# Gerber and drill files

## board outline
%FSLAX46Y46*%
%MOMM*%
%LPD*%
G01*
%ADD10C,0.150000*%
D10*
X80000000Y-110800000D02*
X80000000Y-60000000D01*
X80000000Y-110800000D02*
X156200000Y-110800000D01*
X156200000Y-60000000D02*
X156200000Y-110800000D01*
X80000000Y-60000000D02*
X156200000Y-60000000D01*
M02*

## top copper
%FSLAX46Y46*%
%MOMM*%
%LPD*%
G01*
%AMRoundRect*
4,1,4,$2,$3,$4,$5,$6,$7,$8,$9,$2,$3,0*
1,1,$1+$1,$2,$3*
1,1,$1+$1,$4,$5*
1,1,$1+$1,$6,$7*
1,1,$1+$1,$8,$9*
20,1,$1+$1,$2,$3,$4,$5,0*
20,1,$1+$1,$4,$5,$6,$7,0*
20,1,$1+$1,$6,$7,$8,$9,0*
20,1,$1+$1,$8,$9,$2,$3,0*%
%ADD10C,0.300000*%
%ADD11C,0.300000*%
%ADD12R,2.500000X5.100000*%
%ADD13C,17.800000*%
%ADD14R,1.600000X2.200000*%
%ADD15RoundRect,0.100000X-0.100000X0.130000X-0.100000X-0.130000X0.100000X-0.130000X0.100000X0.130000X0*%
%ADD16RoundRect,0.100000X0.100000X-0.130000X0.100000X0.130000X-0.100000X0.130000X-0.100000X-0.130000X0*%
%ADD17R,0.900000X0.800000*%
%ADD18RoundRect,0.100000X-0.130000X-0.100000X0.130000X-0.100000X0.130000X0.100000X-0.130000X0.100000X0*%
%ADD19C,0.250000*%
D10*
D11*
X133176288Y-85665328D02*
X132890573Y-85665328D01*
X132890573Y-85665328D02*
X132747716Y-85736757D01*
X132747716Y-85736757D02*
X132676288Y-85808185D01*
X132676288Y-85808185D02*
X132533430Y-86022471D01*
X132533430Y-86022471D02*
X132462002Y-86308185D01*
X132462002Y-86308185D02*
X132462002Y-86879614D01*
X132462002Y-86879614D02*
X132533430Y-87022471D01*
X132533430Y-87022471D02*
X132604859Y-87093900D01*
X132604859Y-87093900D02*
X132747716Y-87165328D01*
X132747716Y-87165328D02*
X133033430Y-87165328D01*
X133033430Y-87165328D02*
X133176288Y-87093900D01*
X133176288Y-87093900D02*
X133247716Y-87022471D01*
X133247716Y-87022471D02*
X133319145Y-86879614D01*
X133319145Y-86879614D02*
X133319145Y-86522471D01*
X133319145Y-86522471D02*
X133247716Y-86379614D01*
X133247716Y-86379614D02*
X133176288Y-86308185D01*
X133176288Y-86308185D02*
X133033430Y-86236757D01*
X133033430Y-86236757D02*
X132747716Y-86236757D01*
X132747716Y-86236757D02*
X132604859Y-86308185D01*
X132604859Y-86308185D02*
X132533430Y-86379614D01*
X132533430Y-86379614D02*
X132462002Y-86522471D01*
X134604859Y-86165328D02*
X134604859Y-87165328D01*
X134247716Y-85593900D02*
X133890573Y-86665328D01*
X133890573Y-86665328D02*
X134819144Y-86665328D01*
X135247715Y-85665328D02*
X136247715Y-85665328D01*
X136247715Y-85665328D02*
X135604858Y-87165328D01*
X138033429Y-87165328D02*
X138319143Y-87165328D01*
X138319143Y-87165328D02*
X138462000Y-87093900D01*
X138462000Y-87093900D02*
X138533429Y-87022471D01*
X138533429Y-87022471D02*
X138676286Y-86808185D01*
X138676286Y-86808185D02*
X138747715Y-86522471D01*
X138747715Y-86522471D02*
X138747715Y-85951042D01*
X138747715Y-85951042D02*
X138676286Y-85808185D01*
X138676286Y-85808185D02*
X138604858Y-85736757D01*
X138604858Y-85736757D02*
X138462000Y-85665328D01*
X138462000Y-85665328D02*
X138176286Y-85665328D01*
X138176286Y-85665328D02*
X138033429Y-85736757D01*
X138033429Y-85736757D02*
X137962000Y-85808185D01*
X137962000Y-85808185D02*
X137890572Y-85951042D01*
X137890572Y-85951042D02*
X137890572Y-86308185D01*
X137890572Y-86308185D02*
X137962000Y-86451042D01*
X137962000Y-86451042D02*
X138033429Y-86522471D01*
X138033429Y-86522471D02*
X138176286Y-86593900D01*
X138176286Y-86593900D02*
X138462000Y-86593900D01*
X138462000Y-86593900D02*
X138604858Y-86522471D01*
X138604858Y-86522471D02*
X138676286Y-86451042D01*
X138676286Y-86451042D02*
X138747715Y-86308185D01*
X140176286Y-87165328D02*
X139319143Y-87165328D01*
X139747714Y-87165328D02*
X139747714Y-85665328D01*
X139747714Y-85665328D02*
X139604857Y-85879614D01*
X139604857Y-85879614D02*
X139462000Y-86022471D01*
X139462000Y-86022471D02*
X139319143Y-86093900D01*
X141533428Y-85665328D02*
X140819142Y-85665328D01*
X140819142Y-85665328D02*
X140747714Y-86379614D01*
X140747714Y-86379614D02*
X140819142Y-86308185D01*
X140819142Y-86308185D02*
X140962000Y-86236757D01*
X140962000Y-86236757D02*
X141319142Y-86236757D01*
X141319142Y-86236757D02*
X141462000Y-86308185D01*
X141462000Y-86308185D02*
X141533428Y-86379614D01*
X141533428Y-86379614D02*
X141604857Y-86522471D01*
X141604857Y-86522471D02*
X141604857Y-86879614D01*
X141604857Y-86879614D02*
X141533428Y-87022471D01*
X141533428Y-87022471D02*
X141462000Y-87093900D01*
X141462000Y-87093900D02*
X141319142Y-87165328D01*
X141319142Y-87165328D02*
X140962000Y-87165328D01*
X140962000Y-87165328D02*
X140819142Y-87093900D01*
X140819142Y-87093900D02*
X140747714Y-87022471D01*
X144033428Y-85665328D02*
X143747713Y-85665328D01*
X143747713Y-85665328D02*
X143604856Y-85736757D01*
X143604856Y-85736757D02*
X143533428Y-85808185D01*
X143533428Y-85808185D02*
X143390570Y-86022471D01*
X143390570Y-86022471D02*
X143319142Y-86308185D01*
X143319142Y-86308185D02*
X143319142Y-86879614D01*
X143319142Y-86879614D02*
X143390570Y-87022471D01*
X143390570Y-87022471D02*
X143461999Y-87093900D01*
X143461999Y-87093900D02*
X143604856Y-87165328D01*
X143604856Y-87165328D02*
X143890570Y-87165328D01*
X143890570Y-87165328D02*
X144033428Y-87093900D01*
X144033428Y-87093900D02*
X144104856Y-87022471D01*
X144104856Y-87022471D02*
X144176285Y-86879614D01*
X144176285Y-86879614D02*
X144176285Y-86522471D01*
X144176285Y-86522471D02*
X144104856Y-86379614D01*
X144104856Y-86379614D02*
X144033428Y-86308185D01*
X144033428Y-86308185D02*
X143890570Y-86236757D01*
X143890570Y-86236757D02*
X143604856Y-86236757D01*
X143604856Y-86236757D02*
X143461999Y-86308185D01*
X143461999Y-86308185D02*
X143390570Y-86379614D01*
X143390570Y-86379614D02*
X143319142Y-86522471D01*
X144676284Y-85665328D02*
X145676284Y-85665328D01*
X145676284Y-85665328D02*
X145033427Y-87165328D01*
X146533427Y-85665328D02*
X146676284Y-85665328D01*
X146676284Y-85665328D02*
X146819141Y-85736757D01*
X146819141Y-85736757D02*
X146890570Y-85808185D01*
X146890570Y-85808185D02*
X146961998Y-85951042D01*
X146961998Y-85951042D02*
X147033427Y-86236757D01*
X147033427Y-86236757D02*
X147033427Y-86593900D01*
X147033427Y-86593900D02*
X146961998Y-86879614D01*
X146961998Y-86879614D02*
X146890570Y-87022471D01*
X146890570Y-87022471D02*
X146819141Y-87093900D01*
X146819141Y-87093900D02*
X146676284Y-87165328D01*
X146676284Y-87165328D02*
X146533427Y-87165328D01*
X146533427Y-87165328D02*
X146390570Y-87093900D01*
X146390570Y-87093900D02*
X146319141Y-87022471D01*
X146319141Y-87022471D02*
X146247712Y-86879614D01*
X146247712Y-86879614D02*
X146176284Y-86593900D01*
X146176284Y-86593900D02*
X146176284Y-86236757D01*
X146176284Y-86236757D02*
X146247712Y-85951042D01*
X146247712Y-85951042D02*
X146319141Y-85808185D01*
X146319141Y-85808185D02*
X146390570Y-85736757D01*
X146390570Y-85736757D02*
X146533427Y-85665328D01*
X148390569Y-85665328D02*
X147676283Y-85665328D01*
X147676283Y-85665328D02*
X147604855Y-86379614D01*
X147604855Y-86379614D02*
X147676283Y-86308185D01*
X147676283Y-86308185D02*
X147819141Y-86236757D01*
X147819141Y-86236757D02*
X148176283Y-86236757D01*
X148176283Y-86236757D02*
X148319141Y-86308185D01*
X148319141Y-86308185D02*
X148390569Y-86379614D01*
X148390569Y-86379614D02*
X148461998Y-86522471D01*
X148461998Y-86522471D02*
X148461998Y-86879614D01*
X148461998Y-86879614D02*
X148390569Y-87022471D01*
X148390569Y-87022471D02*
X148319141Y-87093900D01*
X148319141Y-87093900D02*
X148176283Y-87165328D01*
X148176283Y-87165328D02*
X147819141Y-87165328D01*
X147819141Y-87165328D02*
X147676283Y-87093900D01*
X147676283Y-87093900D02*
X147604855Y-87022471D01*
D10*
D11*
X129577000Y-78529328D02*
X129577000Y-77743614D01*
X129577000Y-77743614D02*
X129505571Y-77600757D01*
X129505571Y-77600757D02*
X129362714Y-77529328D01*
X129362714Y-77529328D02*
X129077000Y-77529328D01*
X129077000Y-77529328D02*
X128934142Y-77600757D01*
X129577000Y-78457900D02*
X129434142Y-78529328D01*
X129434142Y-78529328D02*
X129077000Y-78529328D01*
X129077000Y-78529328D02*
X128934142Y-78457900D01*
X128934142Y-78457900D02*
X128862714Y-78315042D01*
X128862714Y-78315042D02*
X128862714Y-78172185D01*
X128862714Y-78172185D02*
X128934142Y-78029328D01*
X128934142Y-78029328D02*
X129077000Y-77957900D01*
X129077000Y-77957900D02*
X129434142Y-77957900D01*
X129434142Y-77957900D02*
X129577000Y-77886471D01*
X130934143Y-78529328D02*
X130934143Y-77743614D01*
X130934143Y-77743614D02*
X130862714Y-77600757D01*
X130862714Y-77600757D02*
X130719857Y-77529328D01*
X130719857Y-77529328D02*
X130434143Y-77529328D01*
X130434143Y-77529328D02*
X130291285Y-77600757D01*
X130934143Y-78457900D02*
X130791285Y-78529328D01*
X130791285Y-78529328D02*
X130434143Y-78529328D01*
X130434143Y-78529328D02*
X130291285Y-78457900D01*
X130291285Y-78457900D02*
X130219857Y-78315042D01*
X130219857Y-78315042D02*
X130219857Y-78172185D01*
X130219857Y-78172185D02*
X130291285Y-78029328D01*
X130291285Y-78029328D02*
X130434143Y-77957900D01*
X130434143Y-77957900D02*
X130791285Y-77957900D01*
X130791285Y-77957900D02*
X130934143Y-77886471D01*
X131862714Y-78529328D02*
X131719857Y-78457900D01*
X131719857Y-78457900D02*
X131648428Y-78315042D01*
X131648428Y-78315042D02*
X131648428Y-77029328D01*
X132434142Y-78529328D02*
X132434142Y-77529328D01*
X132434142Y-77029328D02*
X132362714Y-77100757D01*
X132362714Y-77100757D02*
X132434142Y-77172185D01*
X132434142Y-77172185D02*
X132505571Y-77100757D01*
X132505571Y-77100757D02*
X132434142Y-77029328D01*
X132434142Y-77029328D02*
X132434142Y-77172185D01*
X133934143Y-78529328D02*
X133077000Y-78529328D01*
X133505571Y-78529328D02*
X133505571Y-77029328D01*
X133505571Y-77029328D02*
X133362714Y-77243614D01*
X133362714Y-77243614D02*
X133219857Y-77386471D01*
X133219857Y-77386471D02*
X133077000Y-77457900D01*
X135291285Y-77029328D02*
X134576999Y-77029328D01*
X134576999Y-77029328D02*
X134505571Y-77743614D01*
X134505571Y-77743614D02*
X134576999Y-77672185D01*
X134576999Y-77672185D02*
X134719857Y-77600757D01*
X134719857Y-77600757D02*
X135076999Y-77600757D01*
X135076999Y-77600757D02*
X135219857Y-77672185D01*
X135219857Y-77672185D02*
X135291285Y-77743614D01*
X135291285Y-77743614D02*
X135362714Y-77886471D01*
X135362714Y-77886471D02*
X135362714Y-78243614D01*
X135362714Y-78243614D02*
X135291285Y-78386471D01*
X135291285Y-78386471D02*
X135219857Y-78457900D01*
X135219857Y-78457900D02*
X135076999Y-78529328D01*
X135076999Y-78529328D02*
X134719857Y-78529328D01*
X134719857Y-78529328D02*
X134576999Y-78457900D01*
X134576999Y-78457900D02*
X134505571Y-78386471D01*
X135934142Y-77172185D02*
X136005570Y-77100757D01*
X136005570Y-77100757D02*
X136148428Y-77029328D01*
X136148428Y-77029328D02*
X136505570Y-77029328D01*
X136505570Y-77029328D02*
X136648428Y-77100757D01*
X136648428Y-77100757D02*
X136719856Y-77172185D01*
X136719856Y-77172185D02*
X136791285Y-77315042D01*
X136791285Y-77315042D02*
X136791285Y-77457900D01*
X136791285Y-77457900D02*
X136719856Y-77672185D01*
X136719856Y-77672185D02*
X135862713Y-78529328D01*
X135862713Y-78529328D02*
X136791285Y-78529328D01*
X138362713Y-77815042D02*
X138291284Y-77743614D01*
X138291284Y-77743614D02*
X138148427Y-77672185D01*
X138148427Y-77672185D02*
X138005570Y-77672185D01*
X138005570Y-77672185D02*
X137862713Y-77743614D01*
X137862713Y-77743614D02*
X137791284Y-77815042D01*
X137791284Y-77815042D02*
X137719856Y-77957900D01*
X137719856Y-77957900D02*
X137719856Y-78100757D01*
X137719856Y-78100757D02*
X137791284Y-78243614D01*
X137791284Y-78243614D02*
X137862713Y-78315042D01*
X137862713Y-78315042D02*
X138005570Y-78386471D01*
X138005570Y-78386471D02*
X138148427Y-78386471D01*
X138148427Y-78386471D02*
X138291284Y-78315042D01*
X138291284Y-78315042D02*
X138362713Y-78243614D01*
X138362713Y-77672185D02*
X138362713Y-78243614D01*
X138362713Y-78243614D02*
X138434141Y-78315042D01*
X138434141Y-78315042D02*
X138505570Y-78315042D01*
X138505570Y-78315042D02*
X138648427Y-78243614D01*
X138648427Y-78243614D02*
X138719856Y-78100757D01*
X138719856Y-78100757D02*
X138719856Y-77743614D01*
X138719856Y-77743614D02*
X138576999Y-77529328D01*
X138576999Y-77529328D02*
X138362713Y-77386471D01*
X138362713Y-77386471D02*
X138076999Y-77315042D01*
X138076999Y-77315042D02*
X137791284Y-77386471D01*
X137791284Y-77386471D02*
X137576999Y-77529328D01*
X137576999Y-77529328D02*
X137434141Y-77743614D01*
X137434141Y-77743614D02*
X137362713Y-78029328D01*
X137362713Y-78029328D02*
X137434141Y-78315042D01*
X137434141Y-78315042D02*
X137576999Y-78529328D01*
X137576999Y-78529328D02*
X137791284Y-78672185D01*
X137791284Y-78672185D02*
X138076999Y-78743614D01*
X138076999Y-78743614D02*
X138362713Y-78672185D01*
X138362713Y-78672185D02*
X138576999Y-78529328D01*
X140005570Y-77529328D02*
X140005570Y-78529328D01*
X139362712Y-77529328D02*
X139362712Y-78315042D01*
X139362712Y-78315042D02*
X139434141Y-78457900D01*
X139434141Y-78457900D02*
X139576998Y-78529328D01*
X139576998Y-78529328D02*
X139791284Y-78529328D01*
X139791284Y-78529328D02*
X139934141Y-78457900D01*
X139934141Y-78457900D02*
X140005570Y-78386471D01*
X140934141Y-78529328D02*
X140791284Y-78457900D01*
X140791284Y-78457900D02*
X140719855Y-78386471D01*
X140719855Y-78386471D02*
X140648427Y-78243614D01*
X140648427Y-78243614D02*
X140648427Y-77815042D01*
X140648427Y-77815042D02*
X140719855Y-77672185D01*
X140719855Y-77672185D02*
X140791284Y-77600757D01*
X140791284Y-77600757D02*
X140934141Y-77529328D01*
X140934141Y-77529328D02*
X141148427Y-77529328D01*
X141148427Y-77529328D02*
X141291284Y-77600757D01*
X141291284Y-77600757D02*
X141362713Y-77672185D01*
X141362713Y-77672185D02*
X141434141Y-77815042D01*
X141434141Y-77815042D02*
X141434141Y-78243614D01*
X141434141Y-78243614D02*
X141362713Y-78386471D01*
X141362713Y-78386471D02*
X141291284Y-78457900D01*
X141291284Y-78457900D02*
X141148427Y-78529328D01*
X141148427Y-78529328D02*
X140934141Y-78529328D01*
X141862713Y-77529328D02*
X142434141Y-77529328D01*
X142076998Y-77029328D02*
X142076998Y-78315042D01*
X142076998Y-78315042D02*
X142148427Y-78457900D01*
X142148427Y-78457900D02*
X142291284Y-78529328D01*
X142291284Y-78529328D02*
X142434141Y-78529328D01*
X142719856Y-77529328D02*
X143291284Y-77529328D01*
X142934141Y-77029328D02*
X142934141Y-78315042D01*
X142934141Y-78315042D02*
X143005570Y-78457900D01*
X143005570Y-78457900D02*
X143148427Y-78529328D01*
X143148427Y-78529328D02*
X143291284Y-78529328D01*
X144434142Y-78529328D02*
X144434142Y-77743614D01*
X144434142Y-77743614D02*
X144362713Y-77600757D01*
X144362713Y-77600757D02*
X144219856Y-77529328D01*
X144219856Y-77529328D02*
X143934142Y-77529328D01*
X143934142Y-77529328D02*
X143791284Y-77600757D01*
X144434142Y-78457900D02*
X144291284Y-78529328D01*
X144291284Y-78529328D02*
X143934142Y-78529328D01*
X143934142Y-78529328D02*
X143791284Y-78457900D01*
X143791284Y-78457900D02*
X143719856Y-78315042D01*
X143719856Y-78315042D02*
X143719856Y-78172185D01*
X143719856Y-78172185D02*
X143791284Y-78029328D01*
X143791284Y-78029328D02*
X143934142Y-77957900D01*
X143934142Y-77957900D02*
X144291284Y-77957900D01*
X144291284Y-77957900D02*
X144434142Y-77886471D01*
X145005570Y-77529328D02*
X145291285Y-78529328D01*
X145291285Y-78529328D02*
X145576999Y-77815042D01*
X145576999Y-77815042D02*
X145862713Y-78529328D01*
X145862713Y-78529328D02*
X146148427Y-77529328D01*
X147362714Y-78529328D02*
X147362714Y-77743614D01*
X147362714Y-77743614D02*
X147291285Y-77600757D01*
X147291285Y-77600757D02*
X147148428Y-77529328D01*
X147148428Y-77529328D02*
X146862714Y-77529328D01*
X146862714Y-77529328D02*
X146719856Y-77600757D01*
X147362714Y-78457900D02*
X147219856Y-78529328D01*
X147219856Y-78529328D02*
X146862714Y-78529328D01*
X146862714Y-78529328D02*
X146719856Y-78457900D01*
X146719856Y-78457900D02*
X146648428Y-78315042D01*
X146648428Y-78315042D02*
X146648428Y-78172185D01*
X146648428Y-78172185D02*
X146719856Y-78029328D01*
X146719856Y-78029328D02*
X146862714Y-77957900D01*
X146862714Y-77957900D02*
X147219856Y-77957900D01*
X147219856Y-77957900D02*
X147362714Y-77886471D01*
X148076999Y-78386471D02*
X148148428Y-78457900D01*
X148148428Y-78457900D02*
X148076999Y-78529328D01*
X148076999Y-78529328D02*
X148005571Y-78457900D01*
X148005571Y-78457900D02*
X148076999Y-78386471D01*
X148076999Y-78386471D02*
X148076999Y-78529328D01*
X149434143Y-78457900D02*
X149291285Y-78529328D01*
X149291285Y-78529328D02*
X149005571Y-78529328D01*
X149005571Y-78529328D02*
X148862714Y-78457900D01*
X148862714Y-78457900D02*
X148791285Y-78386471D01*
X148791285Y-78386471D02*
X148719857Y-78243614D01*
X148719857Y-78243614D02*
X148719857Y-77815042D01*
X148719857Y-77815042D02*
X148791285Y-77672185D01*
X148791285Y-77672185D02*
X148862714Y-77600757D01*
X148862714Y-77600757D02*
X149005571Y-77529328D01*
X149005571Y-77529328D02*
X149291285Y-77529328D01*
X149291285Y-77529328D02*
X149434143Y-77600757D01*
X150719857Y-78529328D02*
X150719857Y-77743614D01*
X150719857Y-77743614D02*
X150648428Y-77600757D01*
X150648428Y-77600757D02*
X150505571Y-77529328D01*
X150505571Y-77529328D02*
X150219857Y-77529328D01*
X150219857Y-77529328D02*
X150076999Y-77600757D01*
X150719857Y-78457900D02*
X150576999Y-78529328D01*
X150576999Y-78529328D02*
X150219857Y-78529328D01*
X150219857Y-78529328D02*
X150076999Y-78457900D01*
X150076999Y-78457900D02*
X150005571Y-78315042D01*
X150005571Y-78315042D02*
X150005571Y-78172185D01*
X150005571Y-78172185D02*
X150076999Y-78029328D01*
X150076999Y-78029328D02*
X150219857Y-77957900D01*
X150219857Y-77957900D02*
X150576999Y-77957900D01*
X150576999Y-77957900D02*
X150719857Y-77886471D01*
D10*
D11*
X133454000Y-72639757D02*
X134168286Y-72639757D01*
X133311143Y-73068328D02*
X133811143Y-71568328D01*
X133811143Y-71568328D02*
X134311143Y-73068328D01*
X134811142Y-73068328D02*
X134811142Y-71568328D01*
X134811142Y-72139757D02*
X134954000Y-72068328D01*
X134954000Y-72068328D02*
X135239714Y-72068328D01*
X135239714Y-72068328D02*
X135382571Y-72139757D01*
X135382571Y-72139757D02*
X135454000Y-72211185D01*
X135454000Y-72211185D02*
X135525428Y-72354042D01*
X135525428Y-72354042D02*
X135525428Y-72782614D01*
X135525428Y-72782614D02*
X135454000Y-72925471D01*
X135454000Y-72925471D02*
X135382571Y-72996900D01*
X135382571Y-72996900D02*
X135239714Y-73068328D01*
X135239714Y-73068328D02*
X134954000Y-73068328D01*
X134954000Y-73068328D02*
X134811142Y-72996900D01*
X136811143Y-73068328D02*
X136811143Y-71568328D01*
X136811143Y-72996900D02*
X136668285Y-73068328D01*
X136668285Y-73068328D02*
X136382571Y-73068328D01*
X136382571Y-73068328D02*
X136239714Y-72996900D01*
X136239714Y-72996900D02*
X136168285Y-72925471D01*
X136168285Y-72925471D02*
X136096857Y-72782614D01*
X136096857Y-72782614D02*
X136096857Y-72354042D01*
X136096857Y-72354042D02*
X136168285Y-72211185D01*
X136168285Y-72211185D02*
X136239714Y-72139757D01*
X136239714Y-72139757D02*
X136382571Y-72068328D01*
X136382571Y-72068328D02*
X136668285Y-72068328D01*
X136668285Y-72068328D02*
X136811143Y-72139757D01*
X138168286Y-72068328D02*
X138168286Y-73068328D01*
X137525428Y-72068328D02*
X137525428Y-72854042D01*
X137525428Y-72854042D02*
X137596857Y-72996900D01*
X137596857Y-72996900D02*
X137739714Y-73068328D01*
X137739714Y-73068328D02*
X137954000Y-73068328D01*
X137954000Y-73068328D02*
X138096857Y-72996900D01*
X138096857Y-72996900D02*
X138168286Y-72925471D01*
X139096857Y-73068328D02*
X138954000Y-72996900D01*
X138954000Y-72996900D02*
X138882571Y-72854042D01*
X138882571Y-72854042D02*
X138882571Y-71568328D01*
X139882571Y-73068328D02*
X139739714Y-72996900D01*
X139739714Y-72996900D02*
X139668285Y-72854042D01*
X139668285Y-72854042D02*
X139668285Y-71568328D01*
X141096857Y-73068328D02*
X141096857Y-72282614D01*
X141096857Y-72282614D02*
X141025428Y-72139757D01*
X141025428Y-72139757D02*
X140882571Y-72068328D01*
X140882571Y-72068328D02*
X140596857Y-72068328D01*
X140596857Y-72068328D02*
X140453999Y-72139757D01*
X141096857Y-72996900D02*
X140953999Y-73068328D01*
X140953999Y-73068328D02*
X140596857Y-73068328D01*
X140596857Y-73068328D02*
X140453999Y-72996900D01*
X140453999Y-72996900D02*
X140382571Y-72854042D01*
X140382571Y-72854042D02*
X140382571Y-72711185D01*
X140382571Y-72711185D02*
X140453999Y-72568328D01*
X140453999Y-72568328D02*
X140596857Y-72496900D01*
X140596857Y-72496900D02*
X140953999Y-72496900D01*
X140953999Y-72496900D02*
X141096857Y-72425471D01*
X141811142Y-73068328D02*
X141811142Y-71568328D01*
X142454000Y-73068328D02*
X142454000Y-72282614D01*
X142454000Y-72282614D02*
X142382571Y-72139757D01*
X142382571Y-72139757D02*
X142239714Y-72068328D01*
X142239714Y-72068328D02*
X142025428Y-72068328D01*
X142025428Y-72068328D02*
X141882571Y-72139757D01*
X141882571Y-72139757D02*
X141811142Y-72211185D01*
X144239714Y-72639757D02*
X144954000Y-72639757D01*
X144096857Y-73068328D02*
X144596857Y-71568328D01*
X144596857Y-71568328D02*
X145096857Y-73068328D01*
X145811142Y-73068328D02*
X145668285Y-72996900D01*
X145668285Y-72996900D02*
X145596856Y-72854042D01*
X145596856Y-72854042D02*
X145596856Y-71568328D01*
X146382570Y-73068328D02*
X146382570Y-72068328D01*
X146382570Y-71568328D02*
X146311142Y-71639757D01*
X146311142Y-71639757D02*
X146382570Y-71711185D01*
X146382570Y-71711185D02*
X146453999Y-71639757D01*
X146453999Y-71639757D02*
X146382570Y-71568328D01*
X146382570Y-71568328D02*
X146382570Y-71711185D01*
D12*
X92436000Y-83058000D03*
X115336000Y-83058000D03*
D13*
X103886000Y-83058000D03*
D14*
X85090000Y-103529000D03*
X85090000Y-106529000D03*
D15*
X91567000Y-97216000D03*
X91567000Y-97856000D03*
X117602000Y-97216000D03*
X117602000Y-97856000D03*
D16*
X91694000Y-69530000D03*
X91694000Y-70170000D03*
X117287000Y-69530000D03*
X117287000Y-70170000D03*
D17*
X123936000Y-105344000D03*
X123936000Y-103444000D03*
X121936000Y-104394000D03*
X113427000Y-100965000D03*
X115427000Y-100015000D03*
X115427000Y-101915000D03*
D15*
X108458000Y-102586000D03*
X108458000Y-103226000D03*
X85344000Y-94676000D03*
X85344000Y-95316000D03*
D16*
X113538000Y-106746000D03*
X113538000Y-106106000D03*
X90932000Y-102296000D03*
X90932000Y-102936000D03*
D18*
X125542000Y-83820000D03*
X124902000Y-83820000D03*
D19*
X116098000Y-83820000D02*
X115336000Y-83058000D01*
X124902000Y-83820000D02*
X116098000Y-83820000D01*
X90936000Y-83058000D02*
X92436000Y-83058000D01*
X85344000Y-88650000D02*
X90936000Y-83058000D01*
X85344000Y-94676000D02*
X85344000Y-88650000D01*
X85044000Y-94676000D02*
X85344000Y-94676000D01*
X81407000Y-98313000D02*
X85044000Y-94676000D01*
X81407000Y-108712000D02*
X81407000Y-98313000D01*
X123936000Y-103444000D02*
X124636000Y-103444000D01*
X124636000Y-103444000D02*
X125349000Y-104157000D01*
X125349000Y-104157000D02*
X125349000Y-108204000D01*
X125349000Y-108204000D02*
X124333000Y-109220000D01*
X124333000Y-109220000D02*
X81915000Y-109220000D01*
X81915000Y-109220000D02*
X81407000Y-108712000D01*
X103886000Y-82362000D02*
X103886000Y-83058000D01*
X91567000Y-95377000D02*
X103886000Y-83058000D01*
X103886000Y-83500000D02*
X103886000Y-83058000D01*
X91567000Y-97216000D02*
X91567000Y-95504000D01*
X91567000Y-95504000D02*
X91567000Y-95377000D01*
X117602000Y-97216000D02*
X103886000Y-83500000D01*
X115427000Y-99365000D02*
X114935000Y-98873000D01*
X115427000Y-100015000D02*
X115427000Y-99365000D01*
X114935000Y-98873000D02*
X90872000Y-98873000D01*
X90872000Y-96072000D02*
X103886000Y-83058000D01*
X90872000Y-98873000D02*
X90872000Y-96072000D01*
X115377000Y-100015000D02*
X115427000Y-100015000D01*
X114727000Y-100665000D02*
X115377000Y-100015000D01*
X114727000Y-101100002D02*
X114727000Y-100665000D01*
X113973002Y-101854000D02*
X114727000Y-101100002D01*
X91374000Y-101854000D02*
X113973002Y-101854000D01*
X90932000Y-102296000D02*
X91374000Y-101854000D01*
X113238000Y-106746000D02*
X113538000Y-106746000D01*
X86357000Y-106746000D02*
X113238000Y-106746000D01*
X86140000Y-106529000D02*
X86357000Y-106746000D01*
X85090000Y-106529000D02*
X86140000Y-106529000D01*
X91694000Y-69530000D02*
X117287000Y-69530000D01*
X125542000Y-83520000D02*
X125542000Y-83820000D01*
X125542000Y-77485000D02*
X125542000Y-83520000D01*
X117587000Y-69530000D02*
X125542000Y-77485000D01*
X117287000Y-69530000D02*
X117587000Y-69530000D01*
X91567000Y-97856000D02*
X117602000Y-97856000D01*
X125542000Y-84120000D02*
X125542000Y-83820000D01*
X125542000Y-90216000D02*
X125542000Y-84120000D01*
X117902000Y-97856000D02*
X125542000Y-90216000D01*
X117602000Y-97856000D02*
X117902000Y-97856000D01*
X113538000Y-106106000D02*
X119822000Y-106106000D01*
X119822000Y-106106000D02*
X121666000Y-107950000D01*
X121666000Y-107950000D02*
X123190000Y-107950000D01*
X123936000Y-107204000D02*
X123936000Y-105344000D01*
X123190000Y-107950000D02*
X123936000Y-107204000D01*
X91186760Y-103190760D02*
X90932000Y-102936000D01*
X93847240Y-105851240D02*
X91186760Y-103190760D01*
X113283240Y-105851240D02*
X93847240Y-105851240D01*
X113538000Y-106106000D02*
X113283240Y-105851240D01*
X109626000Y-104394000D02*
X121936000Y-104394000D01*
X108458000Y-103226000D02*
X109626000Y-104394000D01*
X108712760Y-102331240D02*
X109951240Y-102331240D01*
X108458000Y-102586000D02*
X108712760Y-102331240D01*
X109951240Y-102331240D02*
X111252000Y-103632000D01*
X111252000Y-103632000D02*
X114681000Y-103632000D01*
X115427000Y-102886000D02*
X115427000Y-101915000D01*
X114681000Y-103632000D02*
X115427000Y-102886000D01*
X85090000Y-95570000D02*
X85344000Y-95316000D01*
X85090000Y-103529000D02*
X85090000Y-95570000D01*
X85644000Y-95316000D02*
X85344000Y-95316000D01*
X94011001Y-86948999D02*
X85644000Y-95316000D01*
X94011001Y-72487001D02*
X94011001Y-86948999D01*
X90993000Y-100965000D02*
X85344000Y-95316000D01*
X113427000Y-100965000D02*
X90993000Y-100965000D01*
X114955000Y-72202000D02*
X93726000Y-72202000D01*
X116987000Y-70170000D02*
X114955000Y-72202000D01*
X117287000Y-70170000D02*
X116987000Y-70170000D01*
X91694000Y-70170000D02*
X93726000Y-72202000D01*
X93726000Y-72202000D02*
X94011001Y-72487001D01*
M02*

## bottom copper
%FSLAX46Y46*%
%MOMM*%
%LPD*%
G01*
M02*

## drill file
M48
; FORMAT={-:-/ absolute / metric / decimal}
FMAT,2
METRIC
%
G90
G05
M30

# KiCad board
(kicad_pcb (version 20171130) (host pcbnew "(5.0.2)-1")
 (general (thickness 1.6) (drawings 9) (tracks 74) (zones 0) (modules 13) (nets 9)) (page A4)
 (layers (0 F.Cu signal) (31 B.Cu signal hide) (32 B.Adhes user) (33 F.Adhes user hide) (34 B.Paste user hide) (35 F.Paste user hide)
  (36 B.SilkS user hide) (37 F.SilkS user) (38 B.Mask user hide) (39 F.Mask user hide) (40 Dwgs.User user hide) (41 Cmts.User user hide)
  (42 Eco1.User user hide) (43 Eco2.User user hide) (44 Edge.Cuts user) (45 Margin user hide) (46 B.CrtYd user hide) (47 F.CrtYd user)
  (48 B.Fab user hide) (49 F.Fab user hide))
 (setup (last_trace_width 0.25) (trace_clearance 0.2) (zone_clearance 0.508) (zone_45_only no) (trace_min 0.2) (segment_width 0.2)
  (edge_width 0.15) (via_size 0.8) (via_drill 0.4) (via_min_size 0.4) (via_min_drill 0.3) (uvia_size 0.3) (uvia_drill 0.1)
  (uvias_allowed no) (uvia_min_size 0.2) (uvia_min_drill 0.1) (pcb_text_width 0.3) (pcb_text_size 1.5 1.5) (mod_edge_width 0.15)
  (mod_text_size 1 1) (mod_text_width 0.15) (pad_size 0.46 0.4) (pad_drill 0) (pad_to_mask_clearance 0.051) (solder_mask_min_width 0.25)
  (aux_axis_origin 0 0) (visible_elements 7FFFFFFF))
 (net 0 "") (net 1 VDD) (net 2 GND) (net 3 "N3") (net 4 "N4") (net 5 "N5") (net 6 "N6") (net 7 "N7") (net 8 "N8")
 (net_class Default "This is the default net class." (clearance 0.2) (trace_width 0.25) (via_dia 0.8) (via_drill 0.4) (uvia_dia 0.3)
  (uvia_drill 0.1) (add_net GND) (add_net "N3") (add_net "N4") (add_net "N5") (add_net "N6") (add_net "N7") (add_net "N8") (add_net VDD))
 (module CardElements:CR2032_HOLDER (layer F.Cu) (at 103.886 83.058)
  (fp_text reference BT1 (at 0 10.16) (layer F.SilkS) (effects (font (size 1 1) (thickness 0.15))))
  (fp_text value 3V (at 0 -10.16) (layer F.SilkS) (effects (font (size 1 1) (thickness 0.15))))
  (pad 1 smd rect (at -11.45 0) (size 2.5 5.1) (layers F.Cu F.Paste F.Mask) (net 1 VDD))
  (pad 1 smd rect (at 11.45 0) (size 2.5 5.1) (layers F.Cu F.Paste F.Mask) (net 1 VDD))
  (pad 2 smd circle (at 0 0) (size 17.8 17.8) (layers F.Cu F.Paste F.Mask) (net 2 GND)))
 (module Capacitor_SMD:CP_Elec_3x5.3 (layer F.Cu) (at 85.09 105.029 270)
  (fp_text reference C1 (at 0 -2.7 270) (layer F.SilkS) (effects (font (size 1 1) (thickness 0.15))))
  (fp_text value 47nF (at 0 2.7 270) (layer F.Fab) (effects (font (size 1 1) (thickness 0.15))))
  (pad 1 smd rect (at -1.5 0 270) (size 2.2 1.6) (layers F.Cu F.Paste F.Mask) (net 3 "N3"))
  (pad 2 smd rect (at 1.5 0 270) (size 2.2 1.6) (layers F.Cu F.Paste F.Mask) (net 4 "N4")))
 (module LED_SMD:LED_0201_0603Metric (layer F.Cu) (at 91.567 97.536 270)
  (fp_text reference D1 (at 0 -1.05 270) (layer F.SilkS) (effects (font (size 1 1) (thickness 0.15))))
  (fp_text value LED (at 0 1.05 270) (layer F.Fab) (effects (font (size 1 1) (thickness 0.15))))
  (pad "" smd roundrect (at -0.345 0 270) (size 0.318 0.36) (layers F.Paste) (roundrect_rratio 0.25))
  (pad "" smd roundrect (at 0.345 0 270) (size 0.318 0.36) (layers F.Paste) (roundrect_rratio 0.25))
  (pad 1 smd roundrect (at -0.32 0 270) (size 0.46 0.4) (layers F.Cu F.Mask) (roundrect_rratio 0.25) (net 3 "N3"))
  (pad 2 smd roundrect (at 0.32 0 270) (size 0.46 0.4) (layers F.Cu F.Mask) (roundrect_rratio 0.25) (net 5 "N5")))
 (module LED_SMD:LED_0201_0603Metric (layer F.Cu) (at 117.602 97.536 270)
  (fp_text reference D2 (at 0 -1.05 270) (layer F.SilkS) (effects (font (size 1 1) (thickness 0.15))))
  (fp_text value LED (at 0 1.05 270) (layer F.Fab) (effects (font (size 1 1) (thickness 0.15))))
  (pad "" smd roundrect (at -0.345 0 270) (size 0.318 0.36) (layers F.Paste) (roundrect_rratio 0.25))
  (pad "" smd roundrect (at 0.345 0 270) (size 0.318 0.36) (layers F.Paste) (roundrect_rratio 0.25))
  (pad 1 smd roundrect (at -0.32 0 270) (size 0.46 0.4) (layers F.Cu F.Mask) (roundrect_rratio 0.25) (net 3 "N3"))
  (pad 2 smd roundrect (at 0.32 0 270) (size 0.46 0.4) (layers F.Cu F.Mask) (roundrect_rratio 0.25) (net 5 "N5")))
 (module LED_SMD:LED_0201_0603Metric (layer F.Cu) (at 91.694 69.85 90)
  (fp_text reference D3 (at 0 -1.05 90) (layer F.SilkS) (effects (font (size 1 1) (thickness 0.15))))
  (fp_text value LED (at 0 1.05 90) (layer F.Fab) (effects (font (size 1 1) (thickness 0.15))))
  (pad 2 smd roundrect (at 0.32 0 90) (size 0.46 0.4) (layers F.Cu F.Mask) (roundrect_rratio 0.25) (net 5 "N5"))
  (pad 1 smd roundrect (at -0.32 0 90) (size 0.46 0.4) (layers F.Cu F.Mask) (roundrect_rratio 0.25) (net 3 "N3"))
  (pad "" smd roundrect (at 0.345 0 90) (size 0.318 0.36) (layers F.Paste) (roundrect_rratio 0.25))
  (pad "" smd roundrect (at -0.345 0 90) (size 0.318 0.36) (layers F.Paste) (roundrect_rratio 0.25)))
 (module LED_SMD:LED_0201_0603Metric (layer F.Cu) (at 117.287 69.85 90)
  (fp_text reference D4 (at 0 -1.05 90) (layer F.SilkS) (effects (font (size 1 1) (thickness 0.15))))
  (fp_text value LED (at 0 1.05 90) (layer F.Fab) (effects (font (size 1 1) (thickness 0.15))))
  (pad 2 smd roundrect (at 0.32 0 90) (size 0.46 0.4) (layers F.Cu F.Mask) (roundrect_rratio 0.25) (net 5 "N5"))
  (pad 1 smd roundrect (at -0.32 0 90) (size 0.46 0.4) (layers F.Cu F.Mask) (roundrect_rratio 0.25) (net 3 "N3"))
  (pad "" smd roundrect (at 0.345 0 90) (size 0.318 0.36) (layers F.Paste) (roundrect_rratio 0.25))
  (pad "" smd roundrect (at -0.345 0 90) (size 0.318 0.36) (layers F.Paste) (roundrect_rratio 0.25)))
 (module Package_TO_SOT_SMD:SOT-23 (layer F.Cu) (at 122.936 104.394 180)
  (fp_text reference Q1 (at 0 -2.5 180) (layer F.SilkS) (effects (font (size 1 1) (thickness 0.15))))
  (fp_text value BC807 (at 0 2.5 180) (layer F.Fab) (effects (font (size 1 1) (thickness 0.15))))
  (pad 1 smd rect (at -1 -0.95 180) (size 0.9 0.8) (layers F.Cu F.Paste F.Mask) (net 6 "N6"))
  (pad 2 smd rect (at -1 0.95 180) (size 0.9 0.8) (layers F.Cu F.Paste F.Mask) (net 1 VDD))
  (pad 3 smd rect (at 1 0 180) (size 0.9 0.8) (layers F.Cu F.Paste F.Mask) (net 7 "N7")))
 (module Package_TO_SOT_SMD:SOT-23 (layer F.Cu) (at 114.427 100.965 180)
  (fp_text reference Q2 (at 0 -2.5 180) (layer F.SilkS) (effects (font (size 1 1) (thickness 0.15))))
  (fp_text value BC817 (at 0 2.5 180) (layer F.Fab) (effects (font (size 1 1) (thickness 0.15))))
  (pad 3 smd rect (at 1 0 180) (size 0.9 0.8) (layers F.Cu F.Paste F.Mask) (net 3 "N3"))
  (pad 2 smd rect (at -1 0.95 180) (size 0.9 0.8) (layers F.Cu F.Paste F.Mask) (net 2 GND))
  (pad 1 smd rect (at -1 -0.95 180) (size 0.9 0.8) (layers F.Cu F.Paste F.Mask) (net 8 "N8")))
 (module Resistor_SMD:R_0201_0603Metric (layer F.Cu) (at 108.458 102.906 270)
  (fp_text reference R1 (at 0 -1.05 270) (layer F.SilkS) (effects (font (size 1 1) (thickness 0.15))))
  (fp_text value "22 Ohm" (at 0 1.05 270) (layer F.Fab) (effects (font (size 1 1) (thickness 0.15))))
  (pad "" smd roundrect (at -0.345 0 270) (size 0.318 0.36) (layers F.Paste) (roundrect_rratio 0.25))
  (pad "" smd roundrect (at 0.345 0 270) (size 0.318 0.36) (layers F.Paste) (roundrect_rratio 0.25))
  (pad 1 smd roundrect (at -0.32 0 270) (size 0.46 0.4) (layers F.Cu F.Mask) (roundrect_rratio 0.25) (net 8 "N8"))
  (pad 2 smd roundrect (at 0.32 0 270) (size 0.46 0.4) (layers F.Cu F.Mask) (roundrect_rratio 0.25) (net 7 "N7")))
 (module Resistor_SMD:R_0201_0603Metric (layer F.Cu) (at 85.344 94.996 270)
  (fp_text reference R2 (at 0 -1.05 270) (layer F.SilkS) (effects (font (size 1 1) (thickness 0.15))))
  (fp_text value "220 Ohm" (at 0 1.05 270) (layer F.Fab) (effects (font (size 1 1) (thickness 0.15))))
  (pad "" smd roundrect (at -0.345 0 270) (size 0.318 0.36) (layers F.Paste) (roundrect_rratio 0.25))
  (pad "" smd roundrect (at 0.345 0 270) (size 0.318 0.36) (layers F.Paste) (roundrect_rratio 0.25))
  (pad 1 smd roundrect (at -0.32 0 270) (size 0.46 0.4) (layers F.Cu F.Mask) (roundrect_rratio 0.25) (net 1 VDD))
  (pad 2 smd roundrect (at 0.32 0 270) (size 0.46 0.4) (layers F.Cu F.Mask) (roundrect_rratio 0.25) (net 3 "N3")))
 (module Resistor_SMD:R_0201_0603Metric (layer F.Cu) (at 113.538 106.426 90)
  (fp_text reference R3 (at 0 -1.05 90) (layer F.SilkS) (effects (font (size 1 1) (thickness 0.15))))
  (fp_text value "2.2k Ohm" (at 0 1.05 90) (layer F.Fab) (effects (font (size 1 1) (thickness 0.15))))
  (pad "" smd roundrect (at -0.345 0 90) (size 0.318 0.36) (layers F.Paste) (roundrect_rratio 0.25))
  (pad "" smd roundrect (at 0.345 0 90) (size 0.318 0.36) (layers F.Paste) (roundrect_rratio 0.25))
  (pad 1 smd roundrect (at -0.32 0 90) (size 0.46 0.4) (layers F.Cu F.Mask) (roundrect_rratio 0.25) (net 4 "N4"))
  (pad 2 smd roundrect (at 0.32 0 90) (size 0.46 0.4) (layers F.Cu F.Mask) (roundrect_rratio 0.25) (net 6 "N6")))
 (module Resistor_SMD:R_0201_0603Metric (layer F.Cu) (at 90.932 102.616 90)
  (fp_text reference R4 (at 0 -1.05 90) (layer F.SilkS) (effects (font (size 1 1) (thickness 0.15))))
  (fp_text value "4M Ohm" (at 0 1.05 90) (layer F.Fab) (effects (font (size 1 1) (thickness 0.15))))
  (pad 2 smd roundrect (at 0.32 0 90) (size 0.46 0.4) (layers F.Cu F.Mask) (roundrect_rratio 0.25) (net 2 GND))
  (pad 1 smd roundrect (at -0.32 0 90) (size 0.46 0.4) (layers F.Cu F.Mask) (roundrect_rratio 0.25) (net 6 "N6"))
  (pad "" smd roundrect (at 0.345 0 90) (size 0.318 0.36) (layers F.Paste) (roundrect_rratio 0.25))
  (pad "" smd roundrect (at -0.345 0 90) (size 0.318 0.36) (layers F.Paste) (roundrect_rratio 0.25)))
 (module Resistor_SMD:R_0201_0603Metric (layer F.Cu) (at 125.222 83.82)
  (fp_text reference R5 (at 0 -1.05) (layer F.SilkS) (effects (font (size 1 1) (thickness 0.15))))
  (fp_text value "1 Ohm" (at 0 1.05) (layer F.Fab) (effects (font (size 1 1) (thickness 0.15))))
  (pad 2 smd roundrect (at 0.32 0) (size 0.46 0.4) (layers F.Cu F.Mask) (roundrect_rratio 0.25) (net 5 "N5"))
  (pad 1 smd roundrect (at -0.32 0) (size 0.46 0.4) (layers F.Cu F.Mask) (roundrect_rratio 0.25) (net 1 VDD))
  (pad "" smd roundrect (at 0.345 0) (size 0.318 0.36) (layers F.Paste) (roundrect_rratio 0.25))
  (pad "" smd roundrect (at -0.345 0) (size 0.318 0.36) (layers F.Paste) (roundrect_rratio 0.25)))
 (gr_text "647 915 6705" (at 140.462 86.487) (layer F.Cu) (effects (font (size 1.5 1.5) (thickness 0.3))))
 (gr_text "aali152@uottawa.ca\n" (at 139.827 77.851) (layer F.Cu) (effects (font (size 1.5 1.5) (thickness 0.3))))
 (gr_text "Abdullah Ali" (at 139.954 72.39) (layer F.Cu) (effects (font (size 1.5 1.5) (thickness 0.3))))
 (gr_line (start 80 110.8) (end 80 60) (layer Edge.Cuts) (width 0.15))
 (gr_line (start 80 110.8) (end 156.2 110.8) (layer Edge.Cuts) (width 0.15))
 (gr_line (start 156.2 60) (end 156.2 110.8) (layer Edge.Cuts) (width 0.15))
 (gr_line (start 80 60) (end 156.2 60) (layer Edge.Cuts) (width 0.15))
 (segment (start 116.098 83.82) (end 115.336 83.058) (width 0.25) (layer F.Cu) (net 1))
 (segment (start 124.902 83.82) (end 116.098 83.82) (width 0.25) (layer F.Cu) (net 1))
 (segment (start 90.936 83.058) (end 92.436 83.058) (width 0.25) (layer F.Cu) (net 1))
 (segment (start 85.344 88.65) (end 90.936 83.058) (width 0.25) (layer F.Cu) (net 1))
 (segment (start 85.344 94.676) (end 85.344 88.65) (width 0.25) (layer F.Cu) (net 1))
 (segment (start 85.044 94.676) (end 85.344 94.676) (width 0.25) (layer F.Cu) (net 1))
 (segment (start 81.407 98.313) (end 85.044 94.676) (width 0.25) (layer F.Cu) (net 1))
 (segment (start 81.407 108.712) (end 81.407 98.313) (width 0.25) (layer F.Cu) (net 1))
 (segment (start 123.936 103.444) (end 124.636 103.444) (width 0.25) (layer F.Cu) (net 1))
 (segment (start 124.636 103.444) (end 125.349 104.157) (width 0.25) (layer F.Cu) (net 1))
 (segment (start 125.349 104.157) (end 125.349 108.204) (width 0.25) (layer F.Cu) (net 1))
 (segment (start 125.349 108.204) (end 124.333 109.22) (width 0.25) (layer F.Cu) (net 1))
 (segment (start 124.333 109.22) (end 81.915 109.22) (width 0.25) (layer F.Cu) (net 1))
 (segment (start 81.915 109.22) (end 81.407 108.712) (width 0.25) (layer F.Cu) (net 1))
 (segment (start 103.886 82.362) (end 103.886 83.058) (width 0.25) (layer F.Cu) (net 2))
 (segment (start 91.567 95.377) (end 103.886 83.058) (width 0.25) (layer F.Cu) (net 2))
 (segment (start 103.886 83.5) (end 103.886 83.058) (width 0.25) (layer F.Cu) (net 2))
 (segment (start 91.567 97.216) (end 91.567 95.504) (width 0.25) (layer F.Cu) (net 2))
 (segment (start 91.567 95.504) (end 91.567 95.377) (width 0.25) (layer F.Cu) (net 2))
 (segment (start 117.602 97.216) (end 103.886 83.5) (width 0.25) (layer F.Cu) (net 2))
 (segment (start 115.427 99.365) (end 114.935 98.873) (width 0.25) (layer F.Cu) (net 2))
 (segment (start 115.427 100.015) (end 115.427 99.365) (width 0.25) (layer F.Cu) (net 2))
 (segment (start 114.935 98.873) (end 90.872 98.873) (width 0.25) (layer F.Cu) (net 2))
 (segment (start 90.872 96.072) (end 103.886 83.058) (width 0.25) (layer F.Cu) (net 2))
 (segment (start 90.872 98.873) (end 90.872 96.072) (width 0.25) (layer F.Cu) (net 2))
 (segment (start 115.377 100.015) (end 115.427 100.015) (width 0.25) (layer F.Cu) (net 2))
 (segment (start 114.727 100.665) (end 115.377 100.015) (width 0.25) (layer F.Cu) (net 2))
 (segment (start 114.727 101.100002) (end 114.727 100.665) (width 0.25) (layer F.Cu) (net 2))
 (segment (start 113.973002 101.854) (end 114.727 101.100002) (width 0.25) (layer F.Cu) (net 2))
 (segment (start 91.374 101.854) (end 113.973002 101.854) (width 0.25) (layer F.Cu) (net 2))
 (segment (start 90.932 102.296) (end 91.374 101.854) (width 0.25) (layer F.Cu) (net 2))
 (segment (start 113.238 106.746) (end 113.538 106.746) (width 0.25) (layer F.Cu) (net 4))
 (segment (start 86.357 106.746) (end 113.238 106.746) (width 0.25) (layer F.Cu) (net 4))
 (segment (start 86.14 106.529) (end 86.357 106.746) (width 0.25) (layer F.Cu) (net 4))
 (segment (start 85.09 106.529) (end 86.14 106.529) (width 0.25) (layer F.Cu) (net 4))
 (segment (start 91.694 69.53) (end 117.287 69.53) (width 0.25) (layer F.Cu) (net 5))
 (segment (start 125.542 83.52) (end 125.542 83.82) (width 0.25) (layer F.Cu) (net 5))
 (segment (start 125.542 77.485) (end 125.542 83.52) (width 0.25) (layer F.Cu) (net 5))
 (segment (start 117.587 69.53) (end 125.542 77.485) (width 0.25) (layer F.Cu) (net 5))
 (segment (start 117.287 69.53) (end 117.587 69.53) (width 0.25) (layer F.Cu) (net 5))
 (segment (start 91.567 97.856) (end 117.602 97.856) (width 0.25) (layer F.Cu) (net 5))
 (segment (start 125.542 84.12) (end 125.542 83.82) (width 0.25) (layer F.Cu) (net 5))
 (segment (start 125.542 90.216) (end 125.542 84.12) (width 0.25) (layer F.Cu) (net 5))
 (segment (start 117.902 97.856) (end 125.542 90.216) (width 0.25) (layer F.Cu) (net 5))
 (segment (start 117.602 97.856) (end 117.902 97.856) (width 0.25) (layer F.Cu) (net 5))
 (segment (start 113.538 106.106) (end 119.822 106.106) (width 0.25) (layer F.Cu) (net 6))
 (segment (start 119.822 106.106) (end 121.666 107.95) (width 0.25) (layer F.Cu) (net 6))
 (segment (start 121.666 107.95) (end 123.19 107.95) (width 0.25) (layer F.Cu) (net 6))
 (segment (start 123.936 107.204) (end 123.936 105.344) (width 0.25) (layer F.Cu) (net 6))
 (segment (start 123.19 107.95) (end 123.936 107.204) (width 0.25) (layer F.Cu) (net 6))
 (segment (start 91.18676 103.19076) (end 90.932 102.936) (width 0.25) (layer F.Cu) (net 6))
 (segment (start 93.84724 105.85124) (end 91.18676 103.19076) (width 0.25) (layer F.Cu) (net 6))
 (segment (start 113.28324 105.85124) (end 93.84724 105.85124) (width 0.25) (layer F.Cu) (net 6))
 (segment (start 113.538 106.106) (end 113.28324 105.85124) (width 0.25) (layer F.Cu) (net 6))
 (segment (start 109.626 104.394) (end 121.936 104.394) (width 0.25) (layer F.Cu) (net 7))
 (segment (start 108.458 103.226) (end 109.626 104.394) (width 0.25) (layer F.Cu) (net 7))
 (segment (start 108.71276 102.33124) (end 109.95124 102.33124) (width 0.25) (layer F.Cu) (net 8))
 (segment (start 108.458 102.586) (end 108.71276 102.33124) (width 0.25) (layer F.Cu) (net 8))
 (segment (start 109.95124 102.33124) (end 111.252 103.632) (width 0.25) (layer F.Cu) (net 8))
 (segment (start 111.252 103.632) (end 114.681 103.632) (width 0.25) (layer F.Cu) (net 8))
 (segment (start 115.427 102.886) (end 115.427 101.915) (width 0.25) (layer F.Cu) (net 8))
 (segment (start 114.681 103.632) (end 115.427 102.886) (width 0.25) (layer F.Cu) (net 8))
 (segment (start 85.09 95.57) (end 85.344 95.316) (width 0.25) (layer F.Cu) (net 3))
 (segment (start 85.09 103.529) (end 85.09 95.57) (width 0.25) (layer F.Cu) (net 3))
 (segment (start 85.644 95.316) (end 85.344 95.316) (width 0.25) (layer F.Cu) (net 3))
 (segment (start 94.011001 86.948999) (end 85.644 95.316) (width 0.25) (layer F.Cu) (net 3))
 (segment (start 94.011001 72.487001) (end 94.011001 86.948999) (width 0.25) (layer F.Cu) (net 3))
 (segment (start 90.993 100.965) (end 85.344 95.316) (width 0.25) (layer F.Cu) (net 3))
 (segment (start 113.427 100.965) (end 90.993 100.965) (width 0.25) (layer F.Cu) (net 3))
 (segment (start 114.955 72.202) (end 93.726 72.202) (width 0.25) (layer F.Cu) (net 3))
 (segment (start 116.987 70.17) (end 114.955 72.202) (width 0.25) (layer F.Cu) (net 3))
 (segment (start 117.287 70.17) (end 116.987 70.17) (width 0.25) (layer F.Cu) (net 3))
 (segment (start 91.694 70.17) (end 93.726 72.202) (width 0.25) (layer F.Cu) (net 3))
 (segment (start 93.726 72.202) (end 94.011001 72.487001) (width 0.25) (layer F.Cu) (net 3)))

